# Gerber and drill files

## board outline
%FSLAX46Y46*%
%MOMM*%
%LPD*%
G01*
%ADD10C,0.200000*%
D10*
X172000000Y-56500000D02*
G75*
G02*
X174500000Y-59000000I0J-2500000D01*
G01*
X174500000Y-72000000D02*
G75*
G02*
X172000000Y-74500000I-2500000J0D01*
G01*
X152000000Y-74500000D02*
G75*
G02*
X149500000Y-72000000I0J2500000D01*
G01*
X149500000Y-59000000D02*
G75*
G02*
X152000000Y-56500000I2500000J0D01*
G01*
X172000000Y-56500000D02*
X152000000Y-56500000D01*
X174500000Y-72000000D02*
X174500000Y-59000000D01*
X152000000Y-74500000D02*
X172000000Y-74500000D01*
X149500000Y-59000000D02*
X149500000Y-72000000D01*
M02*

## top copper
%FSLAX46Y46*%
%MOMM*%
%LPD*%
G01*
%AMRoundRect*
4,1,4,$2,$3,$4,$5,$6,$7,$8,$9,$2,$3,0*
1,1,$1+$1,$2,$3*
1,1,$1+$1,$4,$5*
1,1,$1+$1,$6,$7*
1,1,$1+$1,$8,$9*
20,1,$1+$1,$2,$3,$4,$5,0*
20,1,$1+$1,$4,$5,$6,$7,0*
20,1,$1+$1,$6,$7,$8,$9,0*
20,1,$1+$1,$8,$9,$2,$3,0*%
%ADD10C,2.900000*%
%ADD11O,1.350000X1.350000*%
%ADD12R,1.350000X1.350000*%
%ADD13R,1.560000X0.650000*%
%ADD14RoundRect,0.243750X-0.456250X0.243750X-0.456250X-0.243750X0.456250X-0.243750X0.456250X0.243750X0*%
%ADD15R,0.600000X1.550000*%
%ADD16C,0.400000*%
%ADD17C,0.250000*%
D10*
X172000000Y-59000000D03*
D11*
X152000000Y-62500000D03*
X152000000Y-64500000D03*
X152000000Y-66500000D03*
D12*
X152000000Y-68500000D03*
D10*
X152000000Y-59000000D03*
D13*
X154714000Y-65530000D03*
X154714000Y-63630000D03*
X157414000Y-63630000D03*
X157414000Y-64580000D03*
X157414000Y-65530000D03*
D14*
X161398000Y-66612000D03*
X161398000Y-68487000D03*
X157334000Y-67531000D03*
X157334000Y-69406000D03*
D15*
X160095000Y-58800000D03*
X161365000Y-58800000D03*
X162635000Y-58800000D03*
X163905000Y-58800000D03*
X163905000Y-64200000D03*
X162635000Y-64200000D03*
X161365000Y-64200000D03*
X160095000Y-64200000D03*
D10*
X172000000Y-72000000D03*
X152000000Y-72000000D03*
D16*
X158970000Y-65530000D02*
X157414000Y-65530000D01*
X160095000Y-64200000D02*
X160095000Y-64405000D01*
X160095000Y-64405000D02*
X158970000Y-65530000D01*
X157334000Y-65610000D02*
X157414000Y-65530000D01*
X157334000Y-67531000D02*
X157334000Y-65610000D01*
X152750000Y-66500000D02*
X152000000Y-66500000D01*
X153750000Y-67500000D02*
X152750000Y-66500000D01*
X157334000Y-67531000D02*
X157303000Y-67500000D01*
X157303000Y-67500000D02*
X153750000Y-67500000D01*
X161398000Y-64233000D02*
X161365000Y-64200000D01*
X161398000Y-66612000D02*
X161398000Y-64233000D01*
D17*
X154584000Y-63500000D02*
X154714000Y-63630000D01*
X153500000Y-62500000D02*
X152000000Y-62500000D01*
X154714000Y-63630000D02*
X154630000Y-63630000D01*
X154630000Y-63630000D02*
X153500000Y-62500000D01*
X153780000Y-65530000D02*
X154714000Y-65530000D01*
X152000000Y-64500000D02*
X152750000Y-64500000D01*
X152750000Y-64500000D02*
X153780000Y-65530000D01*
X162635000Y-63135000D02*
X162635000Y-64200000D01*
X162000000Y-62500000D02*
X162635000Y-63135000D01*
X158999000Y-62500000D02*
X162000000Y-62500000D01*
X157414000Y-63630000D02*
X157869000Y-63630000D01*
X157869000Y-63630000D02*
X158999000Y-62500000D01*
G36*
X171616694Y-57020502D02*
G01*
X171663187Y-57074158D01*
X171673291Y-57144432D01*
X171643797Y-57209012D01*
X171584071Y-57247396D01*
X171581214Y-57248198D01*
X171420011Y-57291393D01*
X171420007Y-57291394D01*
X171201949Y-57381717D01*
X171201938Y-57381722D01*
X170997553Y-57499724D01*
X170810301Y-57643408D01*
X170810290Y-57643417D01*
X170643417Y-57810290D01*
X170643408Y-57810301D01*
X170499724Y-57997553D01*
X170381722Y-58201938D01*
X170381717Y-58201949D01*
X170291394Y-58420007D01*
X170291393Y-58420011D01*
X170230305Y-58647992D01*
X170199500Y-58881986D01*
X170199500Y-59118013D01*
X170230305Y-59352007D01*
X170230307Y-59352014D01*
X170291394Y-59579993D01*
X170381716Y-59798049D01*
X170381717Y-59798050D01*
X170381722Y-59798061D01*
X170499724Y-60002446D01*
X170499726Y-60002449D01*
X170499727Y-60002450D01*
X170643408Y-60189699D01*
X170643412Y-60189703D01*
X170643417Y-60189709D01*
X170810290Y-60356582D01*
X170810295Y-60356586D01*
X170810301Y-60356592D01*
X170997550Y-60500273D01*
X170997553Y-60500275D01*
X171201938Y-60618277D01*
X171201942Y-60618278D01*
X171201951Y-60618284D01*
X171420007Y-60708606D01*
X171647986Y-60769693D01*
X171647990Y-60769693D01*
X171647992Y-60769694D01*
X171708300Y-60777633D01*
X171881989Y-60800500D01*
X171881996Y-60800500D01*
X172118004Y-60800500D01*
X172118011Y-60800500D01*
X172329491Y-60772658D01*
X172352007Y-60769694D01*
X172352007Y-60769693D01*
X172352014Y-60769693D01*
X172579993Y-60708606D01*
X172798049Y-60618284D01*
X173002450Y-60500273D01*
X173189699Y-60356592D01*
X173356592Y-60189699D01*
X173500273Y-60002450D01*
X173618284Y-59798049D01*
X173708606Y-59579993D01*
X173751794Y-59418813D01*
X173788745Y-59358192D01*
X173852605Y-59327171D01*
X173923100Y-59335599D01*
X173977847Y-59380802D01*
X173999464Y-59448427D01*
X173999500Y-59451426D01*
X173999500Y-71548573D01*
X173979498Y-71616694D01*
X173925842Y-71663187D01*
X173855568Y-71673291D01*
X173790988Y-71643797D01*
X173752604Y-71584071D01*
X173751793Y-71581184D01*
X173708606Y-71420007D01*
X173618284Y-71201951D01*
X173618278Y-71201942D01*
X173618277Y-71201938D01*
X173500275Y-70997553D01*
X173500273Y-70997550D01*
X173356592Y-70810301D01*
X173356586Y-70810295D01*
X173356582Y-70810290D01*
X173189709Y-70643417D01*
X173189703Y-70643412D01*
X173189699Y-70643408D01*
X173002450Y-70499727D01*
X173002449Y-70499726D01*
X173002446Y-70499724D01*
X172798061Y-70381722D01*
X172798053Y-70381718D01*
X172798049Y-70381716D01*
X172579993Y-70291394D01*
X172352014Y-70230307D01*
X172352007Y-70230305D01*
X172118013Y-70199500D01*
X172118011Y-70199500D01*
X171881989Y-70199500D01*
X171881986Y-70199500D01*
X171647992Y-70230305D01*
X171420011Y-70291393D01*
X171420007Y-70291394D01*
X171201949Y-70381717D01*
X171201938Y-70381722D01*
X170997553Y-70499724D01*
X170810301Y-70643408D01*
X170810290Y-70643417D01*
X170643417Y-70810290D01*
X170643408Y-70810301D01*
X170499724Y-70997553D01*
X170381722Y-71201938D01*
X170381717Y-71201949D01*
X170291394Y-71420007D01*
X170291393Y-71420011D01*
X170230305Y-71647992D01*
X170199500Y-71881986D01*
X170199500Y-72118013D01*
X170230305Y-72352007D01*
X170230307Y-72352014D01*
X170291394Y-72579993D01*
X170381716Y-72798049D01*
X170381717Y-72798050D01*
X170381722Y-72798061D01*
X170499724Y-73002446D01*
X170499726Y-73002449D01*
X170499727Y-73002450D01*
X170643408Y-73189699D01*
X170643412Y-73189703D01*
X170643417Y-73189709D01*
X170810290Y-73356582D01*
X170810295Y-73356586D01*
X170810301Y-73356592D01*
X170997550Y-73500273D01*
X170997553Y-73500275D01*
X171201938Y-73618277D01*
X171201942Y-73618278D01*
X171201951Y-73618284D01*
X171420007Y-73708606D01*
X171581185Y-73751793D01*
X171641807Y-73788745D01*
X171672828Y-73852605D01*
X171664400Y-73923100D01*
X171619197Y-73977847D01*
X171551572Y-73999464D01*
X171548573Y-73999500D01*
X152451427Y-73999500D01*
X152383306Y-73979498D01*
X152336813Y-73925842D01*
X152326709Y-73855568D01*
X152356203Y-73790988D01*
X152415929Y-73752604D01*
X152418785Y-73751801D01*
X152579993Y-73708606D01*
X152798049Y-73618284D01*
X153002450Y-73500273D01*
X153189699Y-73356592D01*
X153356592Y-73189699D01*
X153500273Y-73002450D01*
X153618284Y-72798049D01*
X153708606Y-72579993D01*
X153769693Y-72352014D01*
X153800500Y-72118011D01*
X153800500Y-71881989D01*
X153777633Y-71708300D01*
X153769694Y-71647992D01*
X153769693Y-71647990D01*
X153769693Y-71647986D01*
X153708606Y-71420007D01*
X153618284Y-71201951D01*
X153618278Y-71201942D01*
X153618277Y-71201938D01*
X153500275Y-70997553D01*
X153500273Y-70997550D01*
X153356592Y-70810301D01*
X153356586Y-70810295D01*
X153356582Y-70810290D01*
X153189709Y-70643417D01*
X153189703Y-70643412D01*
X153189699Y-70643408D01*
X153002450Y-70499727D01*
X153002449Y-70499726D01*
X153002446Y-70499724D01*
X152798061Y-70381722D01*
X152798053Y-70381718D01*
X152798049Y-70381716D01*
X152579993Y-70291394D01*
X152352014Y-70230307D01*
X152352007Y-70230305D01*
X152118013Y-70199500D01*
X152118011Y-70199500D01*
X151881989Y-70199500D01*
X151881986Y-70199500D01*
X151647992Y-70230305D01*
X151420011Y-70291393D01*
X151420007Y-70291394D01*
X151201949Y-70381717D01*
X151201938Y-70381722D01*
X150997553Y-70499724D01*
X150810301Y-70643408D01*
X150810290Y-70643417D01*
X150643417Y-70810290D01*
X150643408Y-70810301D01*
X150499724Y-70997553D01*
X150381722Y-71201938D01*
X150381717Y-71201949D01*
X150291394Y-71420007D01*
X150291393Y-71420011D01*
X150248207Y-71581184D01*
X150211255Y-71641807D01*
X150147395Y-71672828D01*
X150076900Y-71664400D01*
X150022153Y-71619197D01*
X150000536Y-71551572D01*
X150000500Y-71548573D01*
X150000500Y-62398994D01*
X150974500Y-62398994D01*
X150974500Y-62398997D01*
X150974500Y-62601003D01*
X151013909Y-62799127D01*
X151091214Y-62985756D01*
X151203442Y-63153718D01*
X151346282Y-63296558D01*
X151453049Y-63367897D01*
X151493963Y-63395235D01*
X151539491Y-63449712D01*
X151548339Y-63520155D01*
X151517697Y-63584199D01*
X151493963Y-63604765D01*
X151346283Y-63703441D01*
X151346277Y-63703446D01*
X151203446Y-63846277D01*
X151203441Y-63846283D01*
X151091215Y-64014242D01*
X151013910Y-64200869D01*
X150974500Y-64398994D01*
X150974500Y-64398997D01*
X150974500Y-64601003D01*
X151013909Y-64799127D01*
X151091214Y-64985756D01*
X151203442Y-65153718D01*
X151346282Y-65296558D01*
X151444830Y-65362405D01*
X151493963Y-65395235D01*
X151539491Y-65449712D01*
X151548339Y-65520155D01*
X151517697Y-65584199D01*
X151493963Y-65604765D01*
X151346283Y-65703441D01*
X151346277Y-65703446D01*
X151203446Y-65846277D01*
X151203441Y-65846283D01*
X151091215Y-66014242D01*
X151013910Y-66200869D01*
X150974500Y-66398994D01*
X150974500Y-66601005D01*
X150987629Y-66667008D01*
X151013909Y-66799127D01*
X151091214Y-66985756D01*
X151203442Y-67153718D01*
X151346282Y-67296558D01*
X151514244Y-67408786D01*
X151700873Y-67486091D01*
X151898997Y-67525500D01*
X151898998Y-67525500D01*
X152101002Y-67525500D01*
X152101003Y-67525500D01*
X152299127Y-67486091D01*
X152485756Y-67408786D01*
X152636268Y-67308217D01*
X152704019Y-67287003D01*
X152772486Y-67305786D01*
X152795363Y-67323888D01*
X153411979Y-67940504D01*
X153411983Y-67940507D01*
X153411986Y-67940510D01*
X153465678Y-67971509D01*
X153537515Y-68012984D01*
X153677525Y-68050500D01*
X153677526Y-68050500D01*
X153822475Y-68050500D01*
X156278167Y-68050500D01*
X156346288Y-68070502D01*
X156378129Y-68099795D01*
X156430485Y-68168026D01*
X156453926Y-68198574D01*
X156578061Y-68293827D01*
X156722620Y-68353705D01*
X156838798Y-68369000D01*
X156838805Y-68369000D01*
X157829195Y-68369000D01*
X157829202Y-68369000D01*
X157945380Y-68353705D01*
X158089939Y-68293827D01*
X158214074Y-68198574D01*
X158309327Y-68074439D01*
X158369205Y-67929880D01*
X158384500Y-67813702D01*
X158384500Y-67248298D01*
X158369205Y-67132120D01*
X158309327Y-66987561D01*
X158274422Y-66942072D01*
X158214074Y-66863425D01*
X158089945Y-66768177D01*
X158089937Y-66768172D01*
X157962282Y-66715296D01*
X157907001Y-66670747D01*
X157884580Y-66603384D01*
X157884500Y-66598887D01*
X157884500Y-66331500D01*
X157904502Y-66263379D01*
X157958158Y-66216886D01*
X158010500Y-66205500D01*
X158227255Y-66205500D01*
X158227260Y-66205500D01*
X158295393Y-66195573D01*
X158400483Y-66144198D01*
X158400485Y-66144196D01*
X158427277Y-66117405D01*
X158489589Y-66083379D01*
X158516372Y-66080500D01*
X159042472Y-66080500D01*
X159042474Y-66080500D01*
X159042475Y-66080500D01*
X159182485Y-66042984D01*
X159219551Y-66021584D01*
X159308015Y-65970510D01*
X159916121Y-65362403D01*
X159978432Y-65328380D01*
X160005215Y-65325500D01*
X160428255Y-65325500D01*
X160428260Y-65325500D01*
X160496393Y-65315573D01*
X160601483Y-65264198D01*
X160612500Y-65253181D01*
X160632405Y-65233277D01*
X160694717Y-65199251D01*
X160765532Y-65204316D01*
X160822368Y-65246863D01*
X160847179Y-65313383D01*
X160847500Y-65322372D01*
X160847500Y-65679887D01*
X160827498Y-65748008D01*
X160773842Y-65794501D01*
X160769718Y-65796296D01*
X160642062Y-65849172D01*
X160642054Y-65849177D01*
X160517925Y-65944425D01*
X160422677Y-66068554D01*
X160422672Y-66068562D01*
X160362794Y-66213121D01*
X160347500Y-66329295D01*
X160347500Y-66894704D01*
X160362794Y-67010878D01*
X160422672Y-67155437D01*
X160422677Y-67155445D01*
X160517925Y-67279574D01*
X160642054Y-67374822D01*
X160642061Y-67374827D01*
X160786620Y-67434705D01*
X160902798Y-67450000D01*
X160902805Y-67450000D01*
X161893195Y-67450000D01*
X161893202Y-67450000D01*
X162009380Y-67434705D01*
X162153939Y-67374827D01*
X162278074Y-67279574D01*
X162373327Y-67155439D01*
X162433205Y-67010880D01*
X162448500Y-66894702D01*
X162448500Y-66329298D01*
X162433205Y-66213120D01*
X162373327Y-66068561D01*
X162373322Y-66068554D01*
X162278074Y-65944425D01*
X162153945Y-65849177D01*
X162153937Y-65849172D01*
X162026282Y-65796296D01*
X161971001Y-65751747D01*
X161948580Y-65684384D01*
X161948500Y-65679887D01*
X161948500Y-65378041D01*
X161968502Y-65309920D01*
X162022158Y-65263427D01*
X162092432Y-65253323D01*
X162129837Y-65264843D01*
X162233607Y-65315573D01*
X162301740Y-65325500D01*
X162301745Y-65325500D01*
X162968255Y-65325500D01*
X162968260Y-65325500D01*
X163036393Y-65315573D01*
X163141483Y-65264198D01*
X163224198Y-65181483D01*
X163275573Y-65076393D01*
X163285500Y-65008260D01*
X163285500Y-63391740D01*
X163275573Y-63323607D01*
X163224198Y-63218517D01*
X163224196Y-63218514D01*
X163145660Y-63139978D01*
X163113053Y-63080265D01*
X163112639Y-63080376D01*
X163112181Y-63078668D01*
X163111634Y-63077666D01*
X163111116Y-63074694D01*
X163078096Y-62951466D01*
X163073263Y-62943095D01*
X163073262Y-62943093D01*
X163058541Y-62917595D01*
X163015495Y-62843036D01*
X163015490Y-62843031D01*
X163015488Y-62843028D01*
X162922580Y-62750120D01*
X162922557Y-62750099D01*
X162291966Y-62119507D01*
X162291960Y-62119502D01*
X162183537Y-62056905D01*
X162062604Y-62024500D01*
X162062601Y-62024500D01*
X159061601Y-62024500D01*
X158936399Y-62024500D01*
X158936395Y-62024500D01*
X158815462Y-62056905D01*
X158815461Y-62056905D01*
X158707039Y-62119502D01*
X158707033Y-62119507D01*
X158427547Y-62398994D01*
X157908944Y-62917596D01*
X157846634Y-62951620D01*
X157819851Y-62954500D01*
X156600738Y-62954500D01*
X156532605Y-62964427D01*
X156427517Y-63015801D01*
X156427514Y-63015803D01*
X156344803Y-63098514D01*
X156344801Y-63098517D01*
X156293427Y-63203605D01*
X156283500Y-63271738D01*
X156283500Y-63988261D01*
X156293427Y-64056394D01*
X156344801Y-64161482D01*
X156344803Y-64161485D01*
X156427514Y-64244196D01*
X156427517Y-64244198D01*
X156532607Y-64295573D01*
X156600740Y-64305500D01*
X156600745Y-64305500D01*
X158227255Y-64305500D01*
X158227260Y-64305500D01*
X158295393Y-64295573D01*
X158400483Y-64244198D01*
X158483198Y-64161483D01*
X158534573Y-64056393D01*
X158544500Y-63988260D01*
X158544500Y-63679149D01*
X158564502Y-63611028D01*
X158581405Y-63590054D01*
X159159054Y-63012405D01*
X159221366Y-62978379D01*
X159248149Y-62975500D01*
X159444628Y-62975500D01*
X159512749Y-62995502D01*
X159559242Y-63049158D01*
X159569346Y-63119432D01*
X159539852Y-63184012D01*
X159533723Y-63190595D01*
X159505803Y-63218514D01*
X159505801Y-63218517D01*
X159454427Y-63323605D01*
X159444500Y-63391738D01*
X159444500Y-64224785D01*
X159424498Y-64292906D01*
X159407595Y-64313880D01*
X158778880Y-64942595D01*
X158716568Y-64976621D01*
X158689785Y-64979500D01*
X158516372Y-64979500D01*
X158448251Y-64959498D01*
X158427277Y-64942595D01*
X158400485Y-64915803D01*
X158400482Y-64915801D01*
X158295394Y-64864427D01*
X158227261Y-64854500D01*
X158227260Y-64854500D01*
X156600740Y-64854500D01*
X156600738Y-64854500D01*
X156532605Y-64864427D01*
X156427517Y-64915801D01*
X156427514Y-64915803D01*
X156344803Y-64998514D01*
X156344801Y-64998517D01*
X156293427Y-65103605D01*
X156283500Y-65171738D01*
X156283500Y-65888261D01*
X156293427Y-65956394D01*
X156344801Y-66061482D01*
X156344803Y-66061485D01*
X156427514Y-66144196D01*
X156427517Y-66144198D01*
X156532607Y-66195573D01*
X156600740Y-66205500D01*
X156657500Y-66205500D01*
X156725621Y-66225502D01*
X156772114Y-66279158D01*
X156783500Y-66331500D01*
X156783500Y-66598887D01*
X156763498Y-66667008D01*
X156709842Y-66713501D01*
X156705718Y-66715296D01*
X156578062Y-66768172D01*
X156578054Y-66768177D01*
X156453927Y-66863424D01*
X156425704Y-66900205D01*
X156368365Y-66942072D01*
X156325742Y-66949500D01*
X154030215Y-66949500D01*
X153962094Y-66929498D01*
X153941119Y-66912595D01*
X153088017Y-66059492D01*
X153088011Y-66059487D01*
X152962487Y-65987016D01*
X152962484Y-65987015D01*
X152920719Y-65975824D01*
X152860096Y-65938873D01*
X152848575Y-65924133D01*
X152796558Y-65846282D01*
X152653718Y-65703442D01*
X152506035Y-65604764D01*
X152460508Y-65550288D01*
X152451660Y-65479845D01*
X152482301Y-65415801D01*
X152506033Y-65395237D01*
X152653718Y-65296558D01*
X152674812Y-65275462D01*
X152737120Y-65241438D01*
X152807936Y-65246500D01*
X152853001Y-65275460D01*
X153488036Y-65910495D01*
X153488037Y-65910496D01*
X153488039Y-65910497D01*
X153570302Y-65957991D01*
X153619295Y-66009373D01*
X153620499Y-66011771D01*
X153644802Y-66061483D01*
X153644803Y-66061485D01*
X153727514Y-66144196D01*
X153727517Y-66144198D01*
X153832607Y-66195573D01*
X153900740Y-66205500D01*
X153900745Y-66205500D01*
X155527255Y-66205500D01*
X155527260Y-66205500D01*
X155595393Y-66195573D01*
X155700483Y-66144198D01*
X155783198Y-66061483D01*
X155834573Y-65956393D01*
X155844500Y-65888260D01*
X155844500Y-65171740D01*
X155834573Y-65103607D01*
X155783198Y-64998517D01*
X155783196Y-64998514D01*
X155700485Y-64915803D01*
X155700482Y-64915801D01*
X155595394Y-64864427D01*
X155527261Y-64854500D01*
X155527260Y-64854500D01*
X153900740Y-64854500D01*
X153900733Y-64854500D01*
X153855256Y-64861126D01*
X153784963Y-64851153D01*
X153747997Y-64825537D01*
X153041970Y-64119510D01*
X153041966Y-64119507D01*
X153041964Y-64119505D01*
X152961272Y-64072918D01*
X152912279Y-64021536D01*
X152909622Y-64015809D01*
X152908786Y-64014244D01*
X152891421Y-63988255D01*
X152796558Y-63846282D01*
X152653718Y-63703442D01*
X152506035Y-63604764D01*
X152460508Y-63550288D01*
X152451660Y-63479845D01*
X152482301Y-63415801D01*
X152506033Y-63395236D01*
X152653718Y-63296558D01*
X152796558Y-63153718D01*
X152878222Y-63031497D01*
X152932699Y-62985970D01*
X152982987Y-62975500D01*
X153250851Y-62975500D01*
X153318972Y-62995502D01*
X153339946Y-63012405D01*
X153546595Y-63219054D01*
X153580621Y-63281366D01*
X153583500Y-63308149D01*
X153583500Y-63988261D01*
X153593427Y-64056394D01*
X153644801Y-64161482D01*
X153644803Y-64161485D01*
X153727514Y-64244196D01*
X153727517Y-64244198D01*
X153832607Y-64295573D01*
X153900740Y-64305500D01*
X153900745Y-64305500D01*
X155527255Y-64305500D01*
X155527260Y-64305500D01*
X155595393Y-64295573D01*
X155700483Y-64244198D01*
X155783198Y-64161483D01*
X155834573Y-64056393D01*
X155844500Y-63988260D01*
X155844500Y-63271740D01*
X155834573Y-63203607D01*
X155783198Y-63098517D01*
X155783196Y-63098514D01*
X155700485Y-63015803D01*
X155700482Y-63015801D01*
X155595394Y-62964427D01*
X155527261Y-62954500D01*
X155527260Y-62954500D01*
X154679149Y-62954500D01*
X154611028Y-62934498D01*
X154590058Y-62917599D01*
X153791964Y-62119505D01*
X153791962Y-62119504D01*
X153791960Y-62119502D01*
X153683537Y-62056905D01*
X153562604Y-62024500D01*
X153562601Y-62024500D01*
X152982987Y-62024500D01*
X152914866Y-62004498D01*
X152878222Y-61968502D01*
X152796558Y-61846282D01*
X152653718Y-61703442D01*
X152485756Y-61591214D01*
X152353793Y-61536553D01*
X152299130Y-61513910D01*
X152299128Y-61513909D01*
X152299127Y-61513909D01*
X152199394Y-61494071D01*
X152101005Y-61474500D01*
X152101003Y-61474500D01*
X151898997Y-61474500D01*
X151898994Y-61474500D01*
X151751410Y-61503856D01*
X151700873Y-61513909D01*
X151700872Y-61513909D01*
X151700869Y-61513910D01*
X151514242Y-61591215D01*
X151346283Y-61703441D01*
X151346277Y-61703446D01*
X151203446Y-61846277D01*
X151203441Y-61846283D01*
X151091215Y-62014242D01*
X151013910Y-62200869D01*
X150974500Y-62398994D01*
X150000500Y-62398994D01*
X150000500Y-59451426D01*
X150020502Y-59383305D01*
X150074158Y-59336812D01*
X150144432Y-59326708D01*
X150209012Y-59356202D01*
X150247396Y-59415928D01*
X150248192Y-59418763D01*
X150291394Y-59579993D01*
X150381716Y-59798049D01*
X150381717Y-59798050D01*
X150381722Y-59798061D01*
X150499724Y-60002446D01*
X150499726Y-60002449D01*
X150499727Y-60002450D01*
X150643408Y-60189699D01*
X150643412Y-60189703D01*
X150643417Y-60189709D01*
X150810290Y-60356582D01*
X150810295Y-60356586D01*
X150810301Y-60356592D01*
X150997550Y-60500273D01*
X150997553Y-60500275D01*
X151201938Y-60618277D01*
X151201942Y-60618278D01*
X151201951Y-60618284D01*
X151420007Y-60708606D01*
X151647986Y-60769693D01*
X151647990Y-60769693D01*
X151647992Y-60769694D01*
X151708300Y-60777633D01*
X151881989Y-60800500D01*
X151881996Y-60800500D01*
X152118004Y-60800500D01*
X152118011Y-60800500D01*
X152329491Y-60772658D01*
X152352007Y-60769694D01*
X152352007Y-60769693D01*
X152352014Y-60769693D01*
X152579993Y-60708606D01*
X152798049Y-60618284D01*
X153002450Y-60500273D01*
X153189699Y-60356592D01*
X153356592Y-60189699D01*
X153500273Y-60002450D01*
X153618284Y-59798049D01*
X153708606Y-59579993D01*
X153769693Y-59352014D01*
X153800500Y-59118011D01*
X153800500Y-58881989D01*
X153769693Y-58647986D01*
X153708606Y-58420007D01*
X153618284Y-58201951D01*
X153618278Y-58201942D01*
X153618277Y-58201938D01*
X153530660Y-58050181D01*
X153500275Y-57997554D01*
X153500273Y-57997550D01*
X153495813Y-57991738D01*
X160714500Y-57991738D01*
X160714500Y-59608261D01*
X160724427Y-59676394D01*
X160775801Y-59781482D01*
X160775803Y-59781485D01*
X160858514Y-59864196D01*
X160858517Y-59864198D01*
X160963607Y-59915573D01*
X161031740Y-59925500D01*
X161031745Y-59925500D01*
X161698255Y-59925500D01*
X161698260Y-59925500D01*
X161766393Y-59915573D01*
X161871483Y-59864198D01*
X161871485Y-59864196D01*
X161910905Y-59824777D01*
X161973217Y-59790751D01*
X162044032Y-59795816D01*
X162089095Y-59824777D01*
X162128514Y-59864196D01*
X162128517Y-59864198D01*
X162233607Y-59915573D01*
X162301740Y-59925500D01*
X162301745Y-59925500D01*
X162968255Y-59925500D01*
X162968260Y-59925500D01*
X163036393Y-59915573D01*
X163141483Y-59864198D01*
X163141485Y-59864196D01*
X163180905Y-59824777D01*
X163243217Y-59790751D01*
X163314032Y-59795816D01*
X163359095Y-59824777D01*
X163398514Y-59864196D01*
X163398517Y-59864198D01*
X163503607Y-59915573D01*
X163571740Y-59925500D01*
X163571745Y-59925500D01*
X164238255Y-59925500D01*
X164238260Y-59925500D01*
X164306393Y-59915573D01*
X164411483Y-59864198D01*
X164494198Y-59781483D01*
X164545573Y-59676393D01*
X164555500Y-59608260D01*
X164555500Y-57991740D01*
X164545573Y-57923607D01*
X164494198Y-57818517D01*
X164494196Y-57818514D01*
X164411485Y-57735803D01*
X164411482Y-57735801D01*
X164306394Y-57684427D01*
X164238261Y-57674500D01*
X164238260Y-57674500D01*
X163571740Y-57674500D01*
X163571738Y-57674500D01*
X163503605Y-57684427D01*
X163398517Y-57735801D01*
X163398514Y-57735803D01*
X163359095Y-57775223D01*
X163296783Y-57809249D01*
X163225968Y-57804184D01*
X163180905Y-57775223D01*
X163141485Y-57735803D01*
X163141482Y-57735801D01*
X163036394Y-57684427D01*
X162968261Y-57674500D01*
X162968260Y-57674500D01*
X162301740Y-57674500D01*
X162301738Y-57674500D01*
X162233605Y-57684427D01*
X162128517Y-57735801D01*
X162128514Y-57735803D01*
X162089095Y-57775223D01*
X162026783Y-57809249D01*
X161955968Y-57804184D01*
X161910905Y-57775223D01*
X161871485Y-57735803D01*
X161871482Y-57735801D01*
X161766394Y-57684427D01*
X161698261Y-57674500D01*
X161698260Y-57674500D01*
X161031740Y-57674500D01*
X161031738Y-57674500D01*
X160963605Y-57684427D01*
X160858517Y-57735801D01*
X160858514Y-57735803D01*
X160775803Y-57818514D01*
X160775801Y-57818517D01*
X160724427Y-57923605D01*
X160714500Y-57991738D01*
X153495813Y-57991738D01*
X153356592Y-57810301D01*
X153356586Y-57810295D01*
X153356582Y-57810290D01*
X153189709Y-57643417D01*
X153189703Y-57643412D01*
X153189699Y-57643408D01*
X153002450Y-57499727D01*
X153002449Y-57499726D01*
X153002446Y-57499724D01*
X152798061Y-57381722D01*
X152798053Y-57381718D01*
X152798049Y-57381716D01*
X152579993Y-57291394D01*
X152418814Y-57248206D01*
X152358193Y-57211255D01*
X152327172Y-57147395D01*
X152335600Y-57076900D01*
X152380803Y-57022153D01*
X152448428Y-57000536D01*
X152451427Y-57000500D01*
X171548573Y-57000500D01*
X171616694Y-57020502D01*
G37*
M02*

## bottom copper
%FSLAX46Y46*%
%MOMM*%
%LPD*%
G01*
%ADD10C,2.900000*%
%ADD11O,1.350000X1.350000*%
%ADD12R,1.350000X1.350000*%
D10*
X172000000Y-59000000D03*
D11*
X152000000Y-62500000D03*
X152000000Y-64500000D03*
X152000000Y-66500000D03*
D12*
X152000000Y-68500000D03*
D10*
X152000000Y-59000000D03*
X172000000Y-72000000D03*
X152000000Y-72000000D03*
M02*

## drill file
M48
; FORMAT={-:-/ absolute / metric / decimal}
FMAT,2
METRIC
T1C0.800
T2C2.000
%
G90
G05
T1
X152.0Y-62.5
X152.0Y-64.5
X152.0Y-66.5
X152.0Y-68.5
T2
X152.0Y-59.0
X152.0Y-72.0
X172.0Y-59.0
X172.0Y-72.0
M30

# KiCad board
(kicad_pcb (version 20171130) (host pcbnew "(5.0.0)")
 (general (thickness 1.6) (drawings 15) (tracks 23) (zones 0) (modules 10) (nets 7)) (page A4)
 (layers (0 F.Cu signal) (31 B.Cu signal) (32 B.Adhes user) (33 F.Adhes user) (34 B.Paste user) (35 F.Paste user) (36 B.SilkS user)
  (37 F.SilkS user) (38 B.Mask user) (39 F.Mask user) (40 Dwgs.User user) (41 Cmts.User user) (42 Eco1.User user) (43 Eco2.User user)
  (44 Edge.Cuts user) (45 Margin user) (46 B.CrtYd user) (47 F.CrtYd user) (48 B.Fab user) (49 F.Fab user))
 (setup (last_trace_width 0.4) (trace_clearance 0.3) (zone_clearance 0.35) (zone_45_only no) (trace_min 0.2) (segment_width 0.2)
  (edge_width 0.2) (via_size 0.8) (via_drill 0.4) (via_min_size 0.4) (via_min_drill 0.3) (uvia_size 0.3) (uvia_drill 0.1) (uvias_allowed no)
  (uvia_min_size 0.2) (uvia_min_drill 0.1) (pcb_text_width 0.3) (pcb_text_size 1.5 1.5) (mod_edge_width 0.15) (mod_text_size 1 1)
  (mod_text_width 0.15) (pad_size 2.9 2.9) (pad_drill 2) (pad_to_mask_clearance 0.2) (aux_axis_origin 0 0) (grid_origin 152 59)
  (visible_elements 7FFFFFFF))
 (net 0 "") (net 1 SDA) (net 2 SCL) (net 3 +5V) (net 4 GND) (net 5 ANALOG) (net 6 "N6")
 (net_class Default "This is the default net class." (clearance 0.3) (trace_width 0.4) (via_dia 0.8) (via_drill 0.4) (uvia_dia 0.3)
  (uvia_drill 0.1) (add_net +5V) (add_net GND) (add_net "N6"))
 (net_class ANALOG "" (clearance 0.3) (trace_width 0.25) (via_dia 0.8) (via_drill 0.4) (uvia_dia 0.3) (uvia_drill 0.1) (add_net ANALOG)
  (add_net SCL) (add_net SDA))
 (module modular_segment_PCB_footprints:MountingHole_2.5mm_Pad (layer F.Cu) (at 172 61)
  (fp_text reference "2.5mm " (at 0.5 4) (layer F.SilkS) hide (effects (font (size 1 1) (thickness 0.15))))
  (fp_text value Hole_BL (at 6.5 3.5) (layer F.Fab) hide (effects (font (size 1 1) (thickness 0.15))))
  (pad "" np_thru_hole circle (at 0 -2) (size 2.9 2.9) (drill 2) (layers *.Cu *.Mask)))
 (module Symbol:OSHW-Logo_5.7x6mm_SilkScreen (layer F.Cu) (at 169.75 65.75)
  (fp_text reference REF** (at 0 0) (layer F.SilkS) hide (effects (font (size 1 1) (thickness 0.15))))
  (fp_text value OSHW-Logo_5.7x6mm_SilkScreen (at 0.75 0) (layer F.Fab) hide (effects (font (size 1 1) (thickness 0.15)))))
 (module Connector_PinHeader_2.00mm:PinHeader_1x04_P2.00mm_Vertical (layer F.Cu) (at 152 68.5 180)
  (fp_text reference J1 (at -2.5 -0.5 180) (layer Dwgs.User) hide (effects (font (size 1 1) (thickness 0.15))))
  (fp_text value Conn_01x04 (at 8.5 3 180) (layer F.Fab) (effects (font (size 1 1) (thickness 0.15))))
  (pad 4 thru_hole oval (at 0 6 180) (size 1.35 1.35) (drill 0.8) (layers *.Cu *.Mask) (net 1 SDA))
  (pad 3 thru_hole oval (at 0 4 180) (size 1.35 1.35) (drill 0.8) (layers *.Cu *.Mask) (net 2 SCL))
  (pad 2 thru_hole oval (at 0 2 180) (size 1.35 1.35) (drill 0.8) (layers *.Cu *.Mask) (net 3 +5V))
  (pad 1 thru_hole rect (at 0 0 180) (size 1.35 1.35) (drill 0.8) (layers *.Cu *.Mask) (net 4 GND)))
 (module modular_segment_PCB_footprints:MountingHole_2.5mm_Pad (layer F.Cu) (at 152 59)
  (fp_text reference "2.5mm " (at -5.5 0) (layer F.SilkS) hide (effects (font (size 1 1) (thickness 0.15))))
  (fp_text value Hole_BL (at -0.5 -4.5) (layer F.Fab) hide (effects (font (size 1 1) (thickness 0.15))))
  (pad "" np_thru_hole circle (at 0 0) (size 2.9 2.9) (drill 2) (layers *.Cu *.Mask)))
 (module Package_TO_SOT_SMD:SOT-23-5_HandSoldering (layer F.Cu) (at 156.064 64.58 180)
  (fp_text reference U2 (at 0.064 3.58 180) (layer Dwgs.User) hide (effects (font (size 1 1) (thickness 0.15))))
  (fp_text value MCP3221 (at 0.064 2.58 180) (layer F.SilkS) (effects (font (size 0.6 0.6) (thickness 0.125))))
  (pad 5 smd rect (at 1.35 -0.95 180) (size 1.56 0.65) (layers F.Cu F.Paste F.Mask) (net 2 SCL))
  (pad 4 smd rect (at 1.35 0.95 180) (size 1.56 0.65) (layers F.Cu F.Paste F.Mask) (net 1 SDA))
  (pad 3 smd rect (at -1.35 0.95 180) (size 1.56 0.65) (layers F.Cu F.Paste F.Mask) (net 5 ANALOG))
  (pad 2 smd rect (at -1.35 0 180) (size 1.56 0.65) (layers F.Cu F.Paste F.Mask) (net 4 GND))
  (pad 1 smd rect (at -1.35 -0.95 180) (size 1.56 0.65) (layers F.Cu F.Paste F.Mask) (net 3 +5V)))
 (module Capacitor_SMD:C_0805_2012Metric (layer F.Cu) (at 161.398 67.5495 270)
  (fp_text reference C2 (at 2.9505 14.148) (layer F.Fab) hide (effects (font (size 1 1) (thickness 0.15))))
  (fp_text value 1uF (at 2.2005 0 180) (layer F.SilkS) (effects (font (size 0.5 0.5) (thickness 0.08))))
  (pad 1 smd roundrect (at -0.9375 0 270) (size 0.975 1.4) (layers F.Cu F.Paste F.Mask) (roundrect_rratio 0.25) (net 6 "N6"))
  (pad 2 smd roundrect (at 0.9375 0 270) (size 0.975 1.4) (layers F.Cu F.Paste F.Mask) (roundrect_rratio 0.25) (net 4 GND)))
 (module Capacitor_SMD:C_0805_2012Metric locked (layer F.Cu) (at 157.334 68.4685 270)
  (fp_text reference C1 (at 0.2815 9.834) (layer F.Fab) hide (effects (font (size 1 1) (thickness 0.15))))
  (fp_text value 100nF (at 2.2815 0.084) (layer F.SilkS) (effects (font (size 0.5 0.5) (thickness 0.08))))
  (pad 1 smd roundrect (at -0.9375 0 270) (size 0.975 1.4) (layers F.Cu F.Paste F.Mask) (roundrect_rratio 0.25) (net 3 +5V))
  (pad 2 smd roundrect (at 0.9375 0 270) (size 0.975 1.4) (layers F.Cu F.Paste F.Mask) (roundrect_rratio 0.25) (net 4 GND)))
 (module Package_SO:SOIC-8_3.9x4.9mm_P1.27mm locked (layer F.Cu) (at 162 61.5 90)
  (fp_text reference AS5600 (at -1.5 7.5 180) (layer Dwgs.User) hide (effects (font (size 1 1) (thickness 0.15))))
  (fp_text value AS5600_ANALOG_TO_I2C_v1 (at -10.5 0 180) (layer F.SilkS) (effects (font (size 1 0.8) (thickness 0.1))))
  (pad 8 smd rect (at 2.7 -1.905 90) (size 1.55 0.6) (layers F.Cu F.Paste F.Mask) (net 4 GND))
  (pad 7 smd rect (at 2.7 -0.635 90) (size 1.55 0.6) (layers F.Cu F.Paste F.Mask))
  (pad 6 smd rect (at 2.7 0.635 90) (size 1.55 0.6) (layers F.Cu F.Paste F.Mask))
  (pad 5 smd rect (at 2.7 1.905 90) (size 1.55 0.6) (layers F.Cu F.Paste F.Mask))
  (pad 4 smd rect (at -2.7 1.905 90) (size 1.55 0.6) (layers F.Cu F.Paste F.Mask) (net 4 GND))
  (pad 3 smd rect (at -2.7 0.635 90) (size 1.55 0.6) (layers F.Cu F.Paste F.Mask) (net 5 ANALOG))
  (pad 2 smd rect (at -2.7 -0.635 90) (size 1.55 0.6) (layers F.Cu F.Paste F.Mask) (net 6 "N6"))
  (pad 1 smd rect (at -2.7 -1.905 90) (size 1.55 0.6) (layers F.Cu F.Paste F.Mask) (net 3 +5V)))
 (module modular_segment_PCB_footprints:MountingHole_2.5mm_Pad (layer F.Cu) (at 172 74)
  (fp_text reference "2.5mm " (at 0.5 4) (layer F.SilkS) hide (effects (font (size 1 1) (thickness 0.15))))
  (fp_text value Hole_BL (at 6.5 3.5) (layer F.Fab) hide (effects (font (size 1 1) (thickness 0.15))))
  (pad "" np_thru_hole circle (at 0 -2) (size 2.9 2.9) (drill 2) (layers *.Cu *.Mask) (zone_connect 2)))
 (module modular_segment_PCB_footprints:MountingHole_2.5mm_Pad (layer F.Cu) (at 152 74)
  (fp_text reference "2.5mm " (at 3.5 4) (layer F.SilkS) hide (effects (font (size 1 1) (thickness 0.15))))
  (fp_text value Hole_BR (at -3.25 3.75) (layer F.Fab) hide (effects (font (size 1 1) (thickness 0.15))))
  (pad "" np_thru_hole circle (at 0 -2) (size 2.9 2.9) (drill 2) (layers *.Cu *.Mask)))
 (gr_arc (start 172 59) (end 174.5 59) (angle -90) (layer Edge.Cuts) (width 0.2))
 (gr_arc (start 172 72) (end 172 74.5) (angle -90) (layer Edge.Cuts) (width 0.2))
 (gr_arc (start 152 72) (end 149.5 72) (angle -90) (layer Edge.Cuts) (width 0.2))
 (gr_arc (start 152 59) (end 152 56.5) (angle -90) (layer Edge.Cuts) (width 0.2))
 (gr_line (start 172 56.5) (end 152 56.5) (layer Edge.Cuts) (width 0.2))
 (gr_line (start 174.5 72) (end 174.5 59) (layer Edge.Cuts) (width 0.2))
 (gr_line (start 152 74.5) (end 172 74.5) (layer Edge.Cuts) (width 0.2))
 (gr_line (start 149.5 59) (end 149.5 72) (layer Edge.Cuts) (width 0.2))
 (segment (start 158.97 65.53) (end 157.414 65.53) (width 0.4) (layer F.Cu) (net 3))
 (segment (start 160.095 64.2) (end 160.095 64.405) (width 0.4) (layer F.Cu) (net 3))
 (segment (start 160.095 64.405) (end 158.97 65.53) (width 0.4) (layer F.Cu) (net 3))
 (segment (start 157.334 65.61) (end 157.414 65.53) (width 0.4) (layer F.Cu) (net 3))
 (segment (start 157.334 67.531) (end 157.334 65.61) (width 0.4) (layer F.Cu) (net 3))
 (segment (start 152.75 66.5) (end 152 66.5) (width 0.4) (layer F.Cu) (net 3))
 (segment (start 153.75 67.5) (end 152.75 66.5) (width 0.4) (layer F.Cu) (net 3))
 (segment (start 157.334 67.531) (end 157.303 67.5) (width 0.4) (layer F.Cu) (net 3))
 (segment (start 157.303 67.5) (end 153.75 67.5) (width 0.4) (layer F.Cu) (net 3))
 (segment (start 161.398 64.233) (end 161.365 64.2) (width 0.4) (layer F.Cu) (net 6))
 (segment (start 161.398 66.612) (end 161.398 64.233) (width 0.4) (layer F.Cu) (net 6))
 (segment (start 154.584 63.5) (end 154.714 63.63) (width 0.25) (layer F.Cu) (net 1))
 (segment (start 153.5 62.5) (end 152 62.5) (width 0.25) (layer F.Cu) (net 1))
 (segment (start 154.714 63.63) (end 154.63 63.63) (width 0.25) (layer F.Cu) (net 1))
 (segment (start 154.63 63.63) (end 153.5 62.5) (width 0.25) (layer F.Cu) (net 1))
 (segment (start 153.78 65.53) (end 154.714 65.53) (width 0.25) (layer F.Cu) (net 2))
 (segment (start 152 64.5) (end 152.75 64.5) (width 0.25) (layer F.Cu) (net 2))
 (segment (start 152.75 64.5) (end 153.78 65.53) (width 0.25) (layer F.Cu) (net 2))
 (segment (start 162.635 63.135) (end 162.635 64.2) (width 0.25) (layer F.Cu) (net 5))
 (segment (start 162 62.5) (end 162.635 63.135) (width 0.25) (layer F.Cu) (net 5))
 (segment (start 158.999 62.5) (end 162 62.5) (width 0.25) (layer F.Cu) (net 5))
 (segment (start 157.414 63.63) (end 157.869 63.63) (width 0.25) (layer F.Cu) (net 5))
 (segment (start 157.869 63.63) (end 158.999 62.5) (width 0.25) (layer F.Cu) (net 5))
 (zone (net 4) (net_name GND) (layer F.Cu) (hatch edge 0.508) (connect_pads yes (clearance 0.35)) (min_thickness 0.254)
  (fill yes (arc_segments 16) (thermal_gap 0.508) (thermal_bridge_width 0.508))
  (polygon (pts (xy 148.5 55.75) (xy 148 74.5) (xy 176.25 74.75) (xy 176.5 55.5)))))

